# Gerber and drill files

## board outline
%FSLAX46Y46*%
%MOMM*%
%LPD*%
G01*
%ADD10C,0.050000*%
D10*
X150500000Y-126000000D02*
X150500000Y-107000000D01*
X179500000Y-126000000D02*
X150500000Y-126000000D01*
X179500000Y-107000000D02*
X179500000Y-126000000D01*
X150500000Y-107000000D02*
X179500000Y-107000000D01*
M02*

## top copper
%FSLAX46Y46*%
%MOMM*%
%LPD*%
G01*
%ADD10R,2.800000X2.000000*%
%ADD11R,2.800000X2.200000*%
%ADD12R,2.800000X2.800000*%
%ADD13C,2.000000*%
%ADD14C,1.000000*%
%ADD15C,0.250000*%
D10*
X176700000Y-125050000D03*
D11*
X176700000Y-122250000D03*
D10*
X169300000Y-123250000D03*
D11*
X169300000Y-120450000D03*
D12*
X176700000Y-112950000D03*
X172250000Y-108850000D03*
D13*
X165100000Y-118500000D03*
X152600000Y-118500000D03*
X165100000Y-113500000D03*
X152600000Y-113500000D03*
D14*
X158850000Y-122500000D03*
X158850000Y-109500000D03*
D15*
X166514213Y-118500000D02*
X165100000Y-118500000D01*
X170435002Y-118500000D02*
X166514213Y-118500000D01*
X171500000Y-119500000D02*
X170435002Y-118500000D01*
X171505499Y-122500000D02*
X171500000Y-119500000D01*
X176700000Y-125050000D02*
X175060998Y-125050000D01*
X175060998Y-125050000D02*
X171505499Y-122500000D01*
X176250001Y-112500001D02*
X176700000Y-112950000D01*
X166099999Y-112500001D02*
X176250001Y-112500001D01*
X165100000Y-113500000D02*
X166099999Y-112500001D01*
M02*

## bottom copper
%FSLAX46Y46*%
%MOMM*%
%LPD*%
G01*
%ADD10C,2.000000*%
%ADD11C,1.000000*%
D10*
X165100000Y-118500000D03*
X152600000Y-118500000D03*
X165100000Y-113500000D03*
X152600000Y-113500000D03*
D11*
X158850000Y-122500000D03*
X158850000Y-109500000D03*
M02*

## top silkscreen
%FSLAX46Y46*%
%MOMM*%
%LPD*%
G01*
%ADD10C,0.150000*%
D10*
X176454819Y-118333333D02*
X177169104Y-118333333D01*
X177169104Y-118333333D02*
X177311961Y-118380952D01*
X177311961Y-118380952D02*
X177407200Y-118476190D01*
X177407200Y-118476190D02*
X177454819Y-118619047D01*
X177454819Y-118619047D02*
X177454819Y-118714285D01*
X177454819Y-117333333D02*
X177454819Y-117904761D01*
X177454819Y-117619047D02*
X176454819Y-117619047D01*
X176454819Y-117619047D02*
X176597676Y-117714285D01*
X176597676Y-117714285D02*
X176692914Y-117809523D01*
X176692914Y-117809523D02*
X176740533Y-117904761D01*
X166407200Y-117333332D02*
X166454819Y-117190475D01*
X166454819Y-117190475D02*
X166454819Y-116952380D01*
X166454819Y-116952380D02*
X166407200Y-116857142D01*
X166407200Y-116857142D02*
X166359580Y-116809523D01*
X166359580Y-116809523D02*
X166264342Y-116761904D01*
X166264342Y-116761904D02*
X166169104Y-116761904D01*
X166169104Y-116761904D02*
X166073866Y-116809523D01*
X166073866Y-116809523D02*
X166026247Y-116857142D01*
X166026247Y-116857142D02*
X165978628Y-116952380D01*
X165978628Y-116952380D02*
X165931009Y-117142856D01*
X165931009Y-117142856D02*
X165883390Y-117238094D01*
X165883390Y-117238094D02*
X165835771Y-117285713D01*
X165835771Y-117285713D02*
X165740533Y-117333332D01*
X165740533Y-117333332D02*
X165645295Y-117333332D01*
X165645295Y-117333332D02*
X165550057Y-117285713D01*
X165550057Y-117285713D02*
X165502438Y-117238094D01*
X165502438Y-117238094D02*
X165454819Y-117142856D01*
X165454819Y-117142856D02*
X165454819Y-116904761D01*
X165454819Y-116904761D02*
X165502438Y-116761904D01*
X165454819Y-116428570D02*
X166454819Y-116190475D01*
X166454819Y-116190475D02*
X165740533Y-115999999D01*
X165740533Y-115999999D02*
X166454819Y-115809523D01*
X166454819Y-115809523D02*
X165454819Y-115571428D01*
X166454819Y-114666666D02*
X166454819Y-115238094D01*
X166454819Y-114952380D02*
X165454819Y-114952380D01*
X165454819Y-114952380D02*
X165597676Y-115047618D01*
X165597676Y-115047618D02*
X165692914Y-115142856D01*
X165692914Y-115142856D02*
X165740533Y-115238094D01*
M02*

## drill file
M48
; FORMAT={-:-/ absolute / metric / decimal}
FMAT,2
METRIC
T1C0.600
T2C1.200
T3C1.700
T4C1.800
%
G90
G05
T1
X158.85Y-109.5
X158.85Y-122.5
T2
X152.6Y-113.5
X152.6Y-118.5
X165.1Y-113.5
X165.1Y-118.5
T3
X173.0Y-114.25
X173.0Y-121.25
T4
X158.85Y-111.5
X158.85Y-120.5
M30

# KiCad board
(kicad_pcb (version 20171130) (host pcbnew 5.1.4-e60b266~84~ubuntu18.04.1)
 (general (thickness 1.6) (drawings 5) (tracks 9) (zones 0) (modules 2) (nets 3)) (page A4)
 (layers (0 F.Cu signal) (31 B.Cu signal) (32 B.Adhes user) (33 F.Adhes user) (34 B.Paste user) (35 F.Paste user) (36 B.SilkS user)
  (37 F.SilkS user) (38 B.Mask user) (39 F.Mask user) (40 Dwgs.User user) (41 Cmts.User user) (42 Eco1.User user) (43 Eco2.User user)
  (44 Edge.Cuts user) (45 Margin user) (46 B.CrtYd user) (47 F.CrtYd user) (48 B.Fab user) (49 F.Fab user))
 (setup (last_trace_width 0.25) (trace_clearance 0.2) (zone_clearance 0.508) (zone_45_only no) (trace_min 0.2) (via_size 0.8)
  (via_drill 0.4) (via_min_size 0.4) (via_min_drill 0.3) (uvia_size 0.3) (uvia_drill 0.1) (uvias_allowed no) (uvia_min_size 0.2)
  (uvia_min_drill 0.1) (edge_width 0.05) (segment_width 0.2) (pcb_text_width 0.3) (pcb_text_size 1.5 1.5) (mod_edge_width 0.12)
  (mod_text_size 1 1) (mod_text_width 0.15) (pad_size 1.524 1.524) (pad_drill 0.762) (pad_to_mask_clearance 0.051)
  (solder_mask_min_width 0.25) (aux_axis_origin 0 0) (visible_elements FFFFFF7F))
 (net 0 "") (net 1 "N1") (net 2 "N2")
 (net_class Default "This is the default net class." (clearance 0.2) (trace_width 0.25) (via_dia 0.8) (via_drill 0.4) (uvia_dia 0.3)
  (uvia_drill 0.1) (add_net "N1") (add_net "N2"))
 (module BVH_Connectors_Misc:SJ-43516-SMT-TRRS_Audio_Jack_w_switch (layer F.Cu) (at 173 118 90)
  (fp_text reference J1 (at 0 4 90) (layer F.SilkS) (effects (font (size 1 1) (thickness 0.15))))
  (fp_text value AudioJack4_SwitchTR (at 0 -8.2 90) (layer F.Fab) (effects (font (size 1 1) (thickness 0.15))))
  (pad 1 smd rect (at -7.05 3.7 90) (size 2 2.8) (layers F.Cu F.Paste F.Mask) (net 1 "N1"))
  (pad 4 smd rect (at -4.25 3.7 90) (size 2.2 2.8) (layers F.Cu F.Paste F.Mask))
  (pad 6 smd rect (at -5.25 -3.7 90) (size 2 2.8) (layers F.Cu F.Paste F.Mask))
  (pad 3 smd rect (at -2.45 -3.7 90) (size 2.2 2.8) (layers F.Cu F.Paste F.Mask))
  (pad 2 smd rect (at 5.05 3.7 90) (size 2.8 2.8) (layers F.Cu F.Paste F.Mask) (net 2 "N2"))
  (pad 5 smd rect (at 9.15 -0.75 90) (size 2.8 2.8) (layers F.Cu F.Paste F.Mask))
  (pad "" np_thru_hole circle (at -3.25 0 90) (size 1.7 1.7) (drill 1.7) (layers *.Cu *.Mask))
  (pad "" np_thru_hole circle (at 3.75 0 90) (size 1.7 1.7) (drill 1.7) (layers *.Cu *.Mask)))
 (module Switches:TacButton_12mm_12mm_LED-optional (layer F.Cu) (at 158.85 116 180)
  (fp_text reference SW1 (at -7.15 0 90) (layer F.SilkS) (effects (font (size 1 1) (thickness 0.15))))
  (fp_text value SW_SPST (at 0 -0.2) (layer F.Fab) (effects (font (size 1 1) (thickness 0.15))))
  (pad 1 thru_hole circle (at -6.25 -2.5 180) (size 2 2) (drill 1.2) (layers *.Cu *.Mask) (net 1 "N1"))
  (pad 1 thru_hole circle (at 6.25 -2.5 180) (size 2 2) (drill 1.2) (layers *.Cu *.Mask) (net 1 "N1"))
  (pad 2 thru_hole circle (at -6.25 2.5 180) (size 2 2) (drill 1.2) (layers *.Cu *.Mask) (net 2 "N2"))
  (pad 2 thru_hole circle (at 6.25 2.5 180) (size 2 2) (drill 1.2) (layers *.Cu *.Mask) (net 2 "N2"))
  (pad 3 thru_hole circle (at 0 -6.5 180) (size 1 1) (drill 0.6) (layers *.Cu *.Mask))
  (pad 4 thru_hole circle (at 0 6.5 180) (size 1 1) (drill 0.6) (layers *.Cu *.Mask))
  (pad "" np_thru_hole circle (at 0 -4.5 180) (size 1.8 1.8) (drill 1.8) (layers *.Cu *.Mask))
  (pad "" np_thru_hole circle (at 0 4.5 180) (size 1.8 1.8) (drill 1.8) (layers *.Cu *.Mask)))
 (gr_line (start 150.5 126) (end 150.5 107) (layer Edge.Cuts) (width 0.05))
 (gr_line (start 179.5 126) (end 150.5 126) (layer Edge.Cuts) (width 0.05))
 (gr_line (start 179.5 107) (end 179.5 126) (layer Edge.Cuts) (width 0.05))
 (gr_line (start 150.5 107) (end 179.5 107) (layer Edge.Cuts) (width 0.05))
 (segment (start 166.514213 118.5) (end 165.1 118.5) (width 0.25) (layer F.Cu) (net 1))
 (segment (start 170.435002 118.5) (end 166.514213 118.5) (width 0.25) (layer F.Cu) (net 1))
 (segment (start 171.5 119.5) (end 170.435002 118.5) (width 0.25) (layer F.Cu) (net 1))
 (segment (start 171.505499 122.5) (end 171.5 119.5) (width 0.25) (layer F.Cu) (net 1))
 (segment (start 176.7 125.05) (end 175.060998 125.05) (width 0.25) (layer F.Cu) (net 1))
 (segment (start 175.060998 125.05) (end 171.505499 122.5) (width 0.25) (layer F.Cu) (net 1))
 (segment (start 176.250001 112.500001) (end 176.7 112.95) (width 0.25) (layer F.Cu) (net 2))
 (segment (start 166.099999 112.500001) (end 176.250001 112.500001) (width 0.25) (layer F.Cu) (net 2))
 (segment (start 165.1 113.5) (end 166.099999 112.500001) (width 0.25) (layer F.Cu) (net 2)))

